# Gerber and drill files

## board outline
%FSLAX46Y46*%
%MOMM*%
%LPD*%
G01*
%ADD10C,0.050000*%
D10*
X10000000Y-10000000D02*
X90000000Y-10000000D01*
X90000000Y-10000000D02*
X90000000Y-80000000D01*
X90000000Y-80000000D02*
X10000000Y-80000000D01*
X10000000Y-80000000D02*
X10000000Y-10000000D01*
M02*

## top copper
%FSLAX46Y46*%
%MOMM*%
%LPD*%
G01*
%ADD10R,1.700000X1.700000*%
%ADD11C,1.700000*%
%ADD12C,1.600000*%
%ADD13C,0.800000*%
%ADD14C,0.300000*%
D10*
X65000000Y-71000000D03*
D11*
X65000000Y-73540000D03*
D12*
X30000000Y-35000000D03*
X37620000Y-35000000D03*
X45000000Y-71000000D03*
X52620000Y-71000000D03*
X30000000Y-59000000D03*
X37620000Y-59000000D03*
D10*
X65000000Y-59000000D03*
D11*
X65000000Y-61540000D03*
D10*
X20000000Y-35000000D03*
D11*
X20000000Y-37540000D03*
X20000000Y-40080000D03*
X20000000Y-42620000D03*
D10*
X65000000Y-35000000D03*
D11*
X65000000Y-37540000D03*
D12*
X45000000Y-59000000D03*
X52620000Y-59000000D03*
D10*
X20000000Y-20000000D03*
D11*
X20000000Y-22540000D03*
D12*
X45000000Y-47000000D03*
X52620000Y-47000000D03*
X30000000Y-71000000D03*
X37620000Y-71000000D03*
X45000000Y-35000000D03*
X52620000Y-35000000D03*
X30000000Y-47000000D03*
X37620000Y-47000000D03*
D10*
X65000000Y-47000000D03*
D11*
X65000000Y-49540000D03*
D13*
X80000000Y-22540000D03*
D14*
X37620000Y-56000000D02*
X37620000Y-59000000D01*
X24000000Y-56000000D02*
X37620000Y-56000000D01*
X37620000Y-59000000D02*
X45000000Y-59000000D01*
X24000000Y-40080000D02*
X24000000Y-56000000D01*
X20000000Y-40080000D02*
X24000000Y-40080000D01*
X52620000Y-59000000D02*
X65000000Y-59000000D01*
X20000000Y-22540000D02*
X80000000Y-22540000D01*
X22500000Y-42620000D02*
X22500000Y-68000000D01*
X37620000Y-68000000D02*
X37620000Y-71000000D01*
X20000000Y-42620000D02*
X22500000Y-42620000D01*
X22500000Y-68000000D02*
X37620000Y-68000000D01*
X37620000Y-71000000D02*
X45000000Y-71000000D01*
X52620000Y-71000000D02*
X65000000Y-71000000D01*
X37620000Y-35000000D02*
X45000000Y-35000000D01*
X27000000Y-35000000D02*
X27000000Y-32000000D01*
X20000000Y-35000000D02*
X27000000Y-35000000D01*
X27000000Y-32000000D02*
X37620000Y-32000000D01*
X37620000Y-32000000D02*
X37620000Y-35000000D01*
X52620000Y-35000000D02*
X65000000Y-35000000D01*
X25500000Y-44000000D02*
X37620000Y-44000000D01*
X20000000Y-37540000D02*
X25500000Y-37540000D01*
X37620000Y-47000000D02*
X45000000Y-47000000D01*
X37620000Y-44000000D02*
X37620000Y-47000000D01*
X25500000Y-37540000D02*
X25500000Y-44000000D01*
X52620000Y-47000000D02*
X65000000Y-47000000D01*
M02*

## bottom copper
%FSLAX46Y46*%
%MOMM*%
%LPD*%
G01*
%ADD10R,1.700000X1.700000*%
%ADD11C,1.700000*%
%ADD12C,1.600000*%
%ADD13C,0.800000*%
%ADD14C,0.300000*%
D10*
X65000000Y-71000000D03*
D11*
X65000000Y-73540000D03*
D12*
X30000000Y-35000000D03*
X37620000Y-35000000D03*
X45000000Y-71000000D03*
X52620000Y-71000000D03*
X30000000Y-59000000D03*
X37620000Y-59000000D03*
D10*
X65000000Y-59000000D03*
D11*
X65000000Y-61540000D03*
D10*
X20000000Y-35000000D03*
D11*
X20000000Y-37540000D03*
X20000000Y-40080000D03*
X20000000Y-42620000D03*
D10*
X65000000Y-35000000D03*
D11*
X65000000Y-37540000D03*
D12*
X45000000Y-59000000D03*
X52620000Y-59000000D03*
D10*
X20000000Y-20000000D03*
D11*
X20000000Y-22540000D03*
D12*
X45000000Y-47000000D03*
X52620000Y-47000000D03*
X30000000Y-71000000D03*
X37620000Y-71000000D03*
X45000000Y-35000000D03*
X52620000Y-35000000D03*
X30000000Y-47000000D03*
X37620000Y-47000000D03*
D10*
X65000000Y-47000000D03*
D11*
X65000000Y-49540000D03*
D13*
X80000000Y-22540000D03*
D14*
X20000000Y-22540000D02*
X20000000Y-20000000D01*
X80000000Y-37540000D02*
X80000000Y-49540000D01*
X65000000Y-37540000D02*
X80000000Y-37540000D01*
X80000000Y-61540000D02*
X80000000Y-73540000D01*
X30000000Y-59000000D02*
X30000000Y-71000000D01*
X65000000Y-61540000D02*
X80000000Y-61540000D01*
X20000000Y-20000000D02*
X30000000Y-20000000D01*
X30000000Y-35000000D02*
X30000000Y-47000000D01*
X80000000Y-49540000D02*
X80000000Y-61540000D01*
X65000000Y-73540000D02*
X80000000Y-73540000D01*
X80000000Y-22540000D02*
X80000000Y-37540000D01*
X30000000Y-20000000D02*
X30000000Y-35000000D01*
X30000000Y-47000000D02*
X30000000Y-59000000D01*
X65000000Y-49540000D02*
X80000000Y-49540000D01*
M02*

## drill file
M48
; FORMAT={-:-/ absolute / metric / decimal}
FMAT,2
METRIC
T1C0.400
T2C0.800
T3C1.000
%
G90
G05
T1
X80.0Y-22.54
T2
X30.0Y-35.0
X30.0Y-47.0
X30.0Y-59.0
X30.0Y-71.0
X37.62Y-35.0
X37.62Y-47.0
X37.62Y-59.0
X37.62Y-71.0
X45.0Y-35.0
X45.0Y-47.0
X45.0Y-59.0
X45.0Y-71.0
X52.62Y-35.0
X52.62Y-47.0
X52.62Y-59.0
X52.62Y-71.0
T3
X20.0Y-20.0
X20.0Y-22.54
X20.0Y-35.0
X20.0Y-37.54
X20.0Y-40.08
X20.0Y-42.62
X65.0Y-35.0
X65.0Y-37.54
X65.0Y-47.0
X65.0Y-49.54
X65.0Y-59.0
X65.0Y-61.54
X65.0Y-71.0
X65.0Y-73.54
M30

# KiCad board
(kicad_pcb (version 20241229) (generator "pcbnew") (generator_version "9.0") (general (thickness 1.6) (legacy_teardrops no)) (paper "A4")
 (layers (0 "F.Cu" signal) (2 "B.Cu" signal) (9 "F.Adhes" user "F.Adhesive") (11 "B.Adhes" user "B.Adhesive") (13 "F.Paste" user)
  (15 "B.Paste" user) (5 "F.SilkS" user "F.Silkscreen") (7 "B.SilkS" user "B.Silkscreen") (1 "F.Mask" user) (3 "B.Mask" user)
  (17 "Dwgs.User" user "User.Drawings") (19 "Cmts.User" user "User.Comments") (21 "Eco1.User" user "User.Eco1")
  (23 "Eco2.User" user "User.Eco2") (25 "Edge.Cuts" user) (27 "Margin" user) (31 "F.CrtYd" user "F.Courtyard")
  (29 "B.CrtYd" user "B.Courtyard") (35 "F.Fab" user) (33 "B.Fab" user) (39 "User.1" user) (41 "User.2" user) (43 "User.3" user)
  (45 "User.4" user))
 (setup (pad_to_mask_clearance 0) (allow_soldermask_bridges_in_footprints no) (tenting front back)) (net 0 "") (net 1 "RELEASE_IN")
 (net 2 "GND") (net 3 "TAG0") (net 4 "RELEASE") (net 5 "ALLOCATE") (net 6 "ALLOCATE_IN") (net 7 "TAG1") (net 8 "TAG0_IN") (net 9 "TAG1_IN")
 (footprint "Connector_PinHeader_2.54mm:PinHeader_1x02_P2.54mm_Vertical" (layer "F.Cu") (at 65 71)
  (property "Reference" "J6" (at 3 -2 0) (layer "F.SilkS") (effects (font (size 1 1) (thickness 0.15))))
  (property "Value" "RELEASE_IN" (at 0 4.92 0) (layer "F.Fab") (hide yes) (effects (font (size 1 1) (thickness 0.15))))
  (pad "1" thru_hole rect (at 0 0) (size 1.7 1.7) (drill 1) (layers "*.Cu" "*.Mask") (remove_unused_layers no) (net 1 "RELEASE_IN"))
  (pad "2" thru_hole circle (at 0 2.54) (size 1.7 1.7) (drill 1) (layers "*.Cu" "*.Mask") (remove_unused_layers no) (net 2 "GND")))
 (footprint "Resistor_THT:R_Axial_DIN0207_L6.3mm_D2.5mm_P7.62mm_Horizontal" (layer "F.Cu") (at 30 35)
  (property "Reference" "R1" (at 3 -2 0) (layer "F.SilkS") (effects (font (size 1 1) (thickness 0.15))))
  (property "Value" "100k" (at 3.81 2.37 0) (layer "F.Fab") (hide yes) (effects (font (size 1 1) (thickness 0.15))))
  (pad "1" thru_hole circle (at 0 0) (size 1.6 1.6) (drill 0.8) (layers "*.Cu" "*.Mask") (remove_unused_layers no) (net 2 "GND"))
  (pad "2" thru_hole circle (at 7.62 0) (size 1.6 1.6) (drill 0.8) (layers "*.Cu" "*.Mask") (remove_unused_layers no) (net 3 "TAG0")))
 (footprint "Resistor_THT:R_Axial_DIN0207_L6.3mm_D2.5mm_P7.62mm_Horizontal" (layer "F.Cu") (at 45 71)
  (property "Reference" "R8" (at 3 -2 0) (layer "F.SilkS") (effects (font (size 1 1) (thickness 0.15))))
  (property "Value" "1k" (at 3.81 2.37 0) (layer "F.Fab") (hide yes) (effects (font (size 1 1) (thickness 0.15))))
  (pad "1" thru_hole circle (at 0 0) (size 1.6 1.6) (drill 0.8) (layers "*.Cu" "*.Mask") (remove_unused_layers no) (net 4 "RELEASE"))
  (pad "2" thru_hole circle (at 7.62 0) (size 1.6 1.6) (drill 0.8) (layers "*.Cu" "*.Mask") (remove_unused_layers no) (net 1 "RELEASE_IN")))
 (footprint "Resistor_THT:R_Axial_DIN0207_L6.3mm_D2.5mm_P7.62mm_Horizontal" (layer "F.Cu") (at 30 59)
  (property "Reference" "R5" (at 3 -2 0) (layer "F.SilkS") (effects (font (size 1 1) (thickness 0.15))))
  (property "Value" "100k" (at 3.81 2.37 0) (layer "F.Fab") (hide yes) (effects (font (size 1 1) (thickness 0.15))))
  (pad "1" thru_hole circle (at 0 0) (size 1.6 1.6) (drill 0.8) (layers "*.Cu" "*.Mask") (remove_unused_layers no) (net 2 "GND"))
  (pad "2" thru_hole circle (at 7.62 0) (size 1.6 1.6) (drill 0.8) (layers "*.Cu" "*.Mask") (remove_unused_layers no) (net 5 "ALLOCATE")))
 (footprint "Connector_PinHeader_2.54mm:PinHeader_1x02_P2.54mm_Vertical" (layer "F.Cu") (at 65 59)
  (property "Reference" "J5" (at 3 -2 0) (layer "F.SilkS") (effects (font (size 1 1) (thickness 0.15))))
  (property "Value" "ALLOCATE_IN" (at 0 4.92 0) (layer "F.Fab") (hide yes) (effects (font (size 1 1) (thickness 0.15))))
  (pad "1" thru_hole rect (at 0 0) (size 1.7 1.7) (drill 1) (layers "*.Cu" "*.Mask") (remove_unused_layers no) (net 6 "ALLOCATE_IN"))
  (pad "2" thru_hole circle (at 0 2.54) (size 1.7 1.7) (drill 1) (layers "*.Cu" "*.Mask") (remove_unused_layers no) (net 2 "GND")))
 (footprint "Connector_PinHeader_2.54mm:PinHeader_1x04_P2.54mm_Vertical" (layer "F.Cu") (at 20 35)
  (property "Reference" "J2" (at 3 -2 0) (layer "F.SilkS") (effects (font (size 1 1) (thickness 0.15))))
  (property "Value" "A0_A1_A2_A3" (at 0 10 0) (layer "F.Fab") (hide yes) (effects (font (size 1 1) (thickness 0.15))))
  (pad "1" thru_hole rect (at 0 0) (size 1.7 1.7) (drill 1) (layers "*.Cu" "*.Mask") (remove_unused_layers no) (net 3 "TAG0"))
  (pad "2" thru_hole circle (at 0 2.54) (size 1.7 1.7) (drill 1) (layers "*.Cu" "*.Mask") (remove_unused_layers no) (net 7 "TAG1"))
  (pad "3" thru_hole circle (at 0 5.08) (size 1.7 1.7) (drill 1) (layers "*.Cu" "*.Mask") (remove_unused_layers no) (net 5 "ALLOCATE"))
  (pad "4" thru_hole circle (at 0 7.62) (size 1.7 1.7) (drill 1) (layers "*.Cu" "*.Mask") (remove_unused_layers no) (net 4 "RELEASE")))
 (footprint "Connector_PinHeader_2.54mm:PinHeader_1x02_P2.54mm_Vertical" (layer "F.Cu") (at 65 35)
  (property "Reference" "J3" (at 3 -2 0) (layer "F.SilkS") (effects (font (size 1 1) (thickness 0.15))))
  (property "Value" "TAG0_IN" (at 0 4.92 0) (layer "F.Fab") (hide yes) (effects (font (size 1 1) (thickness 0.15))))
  (pad "1" thru_hole rect (at 0 0) (size 1.7 1.7) (drill 1) (layers "*.Cu" "*.Mask") (remove_unused_layers no) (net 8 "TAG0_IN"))
  (pad "2" thru_hole circle (at 0 2.54) (size 1.7 1.7) (drill 1) (layers "*.Cu" "*.Mask") (remove_unused_layers no) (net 2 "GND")))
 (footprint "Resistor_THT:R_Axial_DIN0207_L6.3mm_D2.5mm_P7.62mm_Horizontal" (layer "F.Cu") (at 45 59)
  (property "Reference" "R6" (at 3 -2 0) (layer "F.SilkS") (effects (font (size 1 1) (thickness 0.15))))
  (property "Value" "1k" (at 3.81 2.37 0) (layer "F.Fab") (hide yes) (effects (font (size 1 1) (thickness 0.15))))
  (pad "1" thru_hole circle (at 0 0) (size 1.6 1.6) (drill 0.8) (layers "*.Cu" "*.Mask") (remove_unused_layers no) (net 5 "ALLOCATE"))
  (pad "2" thru_hole circle (at 7.62 0) (size 1.6 1.6) (drill 0.8) (layers "*.Cu" "*.Mask") (remove_unused_layers no) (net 6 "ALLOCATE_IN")))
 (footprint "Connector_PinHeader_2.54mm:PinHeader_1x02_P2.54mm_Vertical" (layer "F.Cu") (at 20 20)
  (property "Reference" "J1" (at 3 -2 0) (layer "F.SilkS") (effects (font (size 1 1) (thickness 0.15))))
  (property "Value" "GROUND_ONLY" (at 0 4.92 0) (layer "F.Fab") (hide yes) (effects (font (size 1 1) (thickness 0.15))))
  (pad "1" thru_hole rect (at 0 0) (size 1.7 1.7) (drill 1) (layers "*.Cu" "*.Mask") (remove_unused_layers no) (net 2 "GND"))
  (pad "2" thru_hole circle (at 0 2.54) (size 1.7 1.7) (drill 1) (layers "*.Cu" "*.Mask") (remove_unused_layers no) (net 2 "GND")))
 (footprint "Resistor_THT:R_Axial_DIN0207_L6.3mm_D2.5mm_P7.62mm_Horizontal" (layer "F.Cu") (at 45 47)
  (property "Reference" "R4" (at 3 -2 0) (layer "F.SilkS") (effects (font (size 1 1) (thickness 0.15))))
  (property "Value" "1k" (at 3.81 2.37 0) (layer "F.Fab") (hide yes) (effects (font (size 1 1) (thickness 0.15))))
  (pad "1" thru_hole circle (at 0 0) (size 1.6 1.6) (drill 0.8) (layers "*.Cu" "*.Mask") (remove_unused_layers no) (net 7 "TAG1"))
  (pad "2" thru_hole circle (at 7.62 0) (size 1.6 1.6) (drill 0.8) (layers "*.Cu" "*.Mask") (remove_unused_layers no) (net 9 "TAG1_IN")))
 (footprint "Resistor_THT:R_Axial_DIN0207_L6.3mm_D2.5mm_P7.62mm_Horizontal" (layer "F.Cu") (at 30 71)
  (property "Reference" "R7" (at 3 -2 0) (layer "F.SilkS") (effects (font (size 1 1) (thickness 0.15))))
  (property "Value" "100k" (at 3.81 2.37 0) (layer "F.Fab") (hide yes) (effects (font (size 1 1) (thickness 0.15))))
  (pad "1" thru_hole circle (at 0 0) (size 1.6 1.6) (drill 0.8) (layers "*.Cu" "*.Mask") (remove_unused_layers no) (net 2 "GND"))
  (pad "2" thru_hole circle (at 7.62 0) (size 1.6 1.6) (drill 0.8) (layers "*.Cu" "*.Mask") (remove_unused_layers no) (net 4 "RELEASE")))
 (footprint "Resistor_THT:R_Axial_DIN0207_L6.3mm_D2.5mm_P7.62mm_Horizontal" (layer "F.Cu") (at 45 35)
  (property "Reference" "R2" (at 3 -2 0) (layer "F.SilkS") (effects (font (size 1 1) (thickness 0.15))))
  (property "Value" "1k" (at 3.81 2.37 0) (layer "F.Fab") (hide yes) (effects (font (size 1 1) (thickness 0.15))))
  (pad "1" thru_hole circle (at 0 0) (size 1.6 1.6) (drill 0.8) (layers "*.Cu" "*.Mask") (remove_unused_layers no) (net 3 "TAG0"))
  (pad "2" thru_hole circle (at 7.62 0) (size 1.6 1.6) (drill 0.8) (layers "*.Cu" "*.Mask") (remove_unused_layers no) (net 8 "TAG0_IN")))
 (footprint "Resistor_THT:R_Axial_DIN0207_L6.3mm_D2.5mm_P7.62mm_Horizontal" (layer "F.Cu") (at 30 47)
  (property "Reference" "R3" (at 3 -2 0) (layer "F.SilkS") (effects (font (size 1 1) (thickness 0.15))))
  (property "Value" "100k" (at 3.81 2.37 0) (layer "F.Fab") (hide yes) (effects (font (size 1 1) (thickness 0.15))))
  (pad "1" thru_hole circle (at 0 0) (size 1.6 1.6) (drill 0.8) (layers "*.Cu" "*.Mask") (remove_unused_layers no) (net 2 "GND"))
  (pad "2" thru_hole circle (at 7.62 0) (size 1.6 1.6) (drill 0.8) (layers "*.Cu" "*.Mask") (remove_unused_layers no) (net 7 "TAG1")))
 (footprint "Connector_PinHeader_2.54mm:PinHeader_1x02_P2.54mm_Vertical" (layer "F.Cu") (at 65 47)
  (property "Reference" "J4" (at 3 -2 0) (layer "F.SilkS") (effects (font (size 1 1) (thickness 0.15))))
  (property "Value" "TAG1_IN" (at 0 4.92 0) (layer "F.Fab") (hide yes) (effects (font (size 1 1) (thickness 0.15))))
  (pad "1" thru_hole rect (at 0 0) (size 1.7 1.7) (drill 1) (layers "*.Cu" "*.Mask") (remove_unused_layers no) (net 9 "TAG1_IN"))
  (pad "2" thru_hole circle (at 0 2.54) (size 1.7 1.7) (drill 1) (layers "*.Cu" "*.Mask") (remove_unused_layers no) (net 2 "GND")))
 (gr_line (start 10 10) (end 90 10) (stroke (width 0.05) (type default)) (layer "Edge.Cuts"))
 (gr_line (start 90 10) (end 90 80) (stroke (width 0.05) (type default)) (layer "Edge.Cuts"))
 (gr_line (start 90 80) (end 10 80) (stroke (width 0.05) (type default)) (layer "Edge.Cuts"))
 (gr_line (start 10 80) (end 10 10) (stroke (width 0.05) (type default)) (layer "Edge.Cuts"))
 (segment (start 37.62 56) (end 37.62 59) (width 0.3) (layer "F.Cu") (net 5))
 (segment (start 24 56) (end 37.62 56) (width 0.3) (layer "F.Cu") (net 5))
 (segment (start 37.62 59) (end 45 59) (width 0.3) (layer "F.Cu") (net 5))
 (segment (start 24 40.08) (end 24 56) (width 0.3) (layer "F.Cu") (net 5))
 (segment (start 20 40.08) (end 24 40.08) (width 0.3) (layer "F.Cu") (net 5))
 (segment (start 52.62 59) (end 65 59) (width 0.3) (layer "F.Cu") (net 6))
 (segment (start 20 22.54) (end 80 22.54) (width 0.3) (layer "F.Cu") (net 2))
 (via (at 80 22.54) (size 0.8) (drill 0.4) (layers "F.Cu" "B.Cu") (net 2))
 (segment (start 20 22.54) (end 20 20) (width 0.3) (layer "B.Cu") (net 2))
 (segment (start 80 37.54) (end 80 49.54) (width 0.3) (layer "B.Cu") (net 2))
 (segment (start 65 37.54) (end 80 37.54) (width 0.3) (layer "B.Cu") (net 2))
 (segment (start 80 61.54) (end 80 73.54) (width 0.3) (layer "B.Cu") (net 2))
 (segment (start 30 59) (end 30 71) (width 0.3) (layer "B.Cu") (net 2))
 (segment (start 65 61.54) (end 80 61.54) (width 0.3) (layer "B.Cu") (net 2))
 (segment (start 20 20) (end 30 20) (width 0.3) (layer "B.Cu") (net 2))
 (segment (start 30 35) (end 30 47) (width 0.3) (layer "B.Cu") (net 2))
 (segment (start 80 49.54) (end 80 61.54) (width 0.3) (layer "B.Cu") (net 2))
 (segment (start 65 73.54) (end 80 73.54) (width 0.3) (layer "B.Cu") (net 2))
 (segment (start 80 22.54) (end 80 37.54) (width 0.3) (layer "B.Cu") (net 2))
 (segment (start 30 20) (end 30 35) (width 0.3) (layer "B.Cu") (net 2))
 (segment (start 30 47) (end 30 59) (width 0.3) (layer "B.Cu") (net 2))
 (segment (start 65 49.54) (end 80 49.54) (width 0.3) (layer "B.Cu") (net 2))
 (segment (start 22.5 42.62) (end 22.5 68) (width 0.3) (layer "F.Cu") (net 4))
 (segment (start 37.62 68) (end 37.62 71) (width 0.3) (layer "F.Cu") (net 4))
 (segment (start 20 42.62) (end 22.5 42.62) (width 0.3) (layer "F.Cu") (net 4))
 (segment (start 22.5 68) (end 37.62 68) (width 0.3) (layer "F.Cu") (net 4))
 (segment (start 37.62 71) (end 45 71) (width 0.3) (layer "F.Cu") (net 4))
 (segment (start 52.62 71) (end 65 71) (width 0.3) (layer "F.Cu") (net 1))
 (segment (start 37.62 35) (end 45 35) (width 0.3) (layer "F.Cu") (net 3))
 (segment (start 27 35) (end 27 32) (width 0.3) (layer "F.Cu") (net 3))
 (segment (start 20 35) (end 27 35) (width 0.3) (layer "F.Cu") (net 3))
 (segment (start 27 32) (end 37.62 32) (width 0.3) (layer "F.Cu") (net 3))
 (segment (start 37.62 32) (end 37.62 35) (width 0.3) (layer "F.Cu") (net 3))
 (segment (start 52.62 35) (end 65 35) (width 0.3) (layer "F.Cu") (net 8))
 (segment (start 25.5 44) (end 37.62 44) (width 0.3) (layer "F.Cu") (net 7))
 (segment (start 20 37.54) (end 25.5 37.54) (width 0.3) (layer "F.Cu") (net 7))
 (segment (start 37.62 47) (end 45 47) (width 0.3) (layer "F.Cu") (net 7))
 (segment (start 37.62 44) (end 37.62 47) (width 0.3) (layer "F.Cu") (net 7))
 (segment (start 25.5 37.54) (end 25.5 44) (width 0.3) (layer "F.Cu") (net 7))
 (segment (start 52.62 47) (end 65 47) (width 0.3) (layer "F.Cu") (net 9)))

